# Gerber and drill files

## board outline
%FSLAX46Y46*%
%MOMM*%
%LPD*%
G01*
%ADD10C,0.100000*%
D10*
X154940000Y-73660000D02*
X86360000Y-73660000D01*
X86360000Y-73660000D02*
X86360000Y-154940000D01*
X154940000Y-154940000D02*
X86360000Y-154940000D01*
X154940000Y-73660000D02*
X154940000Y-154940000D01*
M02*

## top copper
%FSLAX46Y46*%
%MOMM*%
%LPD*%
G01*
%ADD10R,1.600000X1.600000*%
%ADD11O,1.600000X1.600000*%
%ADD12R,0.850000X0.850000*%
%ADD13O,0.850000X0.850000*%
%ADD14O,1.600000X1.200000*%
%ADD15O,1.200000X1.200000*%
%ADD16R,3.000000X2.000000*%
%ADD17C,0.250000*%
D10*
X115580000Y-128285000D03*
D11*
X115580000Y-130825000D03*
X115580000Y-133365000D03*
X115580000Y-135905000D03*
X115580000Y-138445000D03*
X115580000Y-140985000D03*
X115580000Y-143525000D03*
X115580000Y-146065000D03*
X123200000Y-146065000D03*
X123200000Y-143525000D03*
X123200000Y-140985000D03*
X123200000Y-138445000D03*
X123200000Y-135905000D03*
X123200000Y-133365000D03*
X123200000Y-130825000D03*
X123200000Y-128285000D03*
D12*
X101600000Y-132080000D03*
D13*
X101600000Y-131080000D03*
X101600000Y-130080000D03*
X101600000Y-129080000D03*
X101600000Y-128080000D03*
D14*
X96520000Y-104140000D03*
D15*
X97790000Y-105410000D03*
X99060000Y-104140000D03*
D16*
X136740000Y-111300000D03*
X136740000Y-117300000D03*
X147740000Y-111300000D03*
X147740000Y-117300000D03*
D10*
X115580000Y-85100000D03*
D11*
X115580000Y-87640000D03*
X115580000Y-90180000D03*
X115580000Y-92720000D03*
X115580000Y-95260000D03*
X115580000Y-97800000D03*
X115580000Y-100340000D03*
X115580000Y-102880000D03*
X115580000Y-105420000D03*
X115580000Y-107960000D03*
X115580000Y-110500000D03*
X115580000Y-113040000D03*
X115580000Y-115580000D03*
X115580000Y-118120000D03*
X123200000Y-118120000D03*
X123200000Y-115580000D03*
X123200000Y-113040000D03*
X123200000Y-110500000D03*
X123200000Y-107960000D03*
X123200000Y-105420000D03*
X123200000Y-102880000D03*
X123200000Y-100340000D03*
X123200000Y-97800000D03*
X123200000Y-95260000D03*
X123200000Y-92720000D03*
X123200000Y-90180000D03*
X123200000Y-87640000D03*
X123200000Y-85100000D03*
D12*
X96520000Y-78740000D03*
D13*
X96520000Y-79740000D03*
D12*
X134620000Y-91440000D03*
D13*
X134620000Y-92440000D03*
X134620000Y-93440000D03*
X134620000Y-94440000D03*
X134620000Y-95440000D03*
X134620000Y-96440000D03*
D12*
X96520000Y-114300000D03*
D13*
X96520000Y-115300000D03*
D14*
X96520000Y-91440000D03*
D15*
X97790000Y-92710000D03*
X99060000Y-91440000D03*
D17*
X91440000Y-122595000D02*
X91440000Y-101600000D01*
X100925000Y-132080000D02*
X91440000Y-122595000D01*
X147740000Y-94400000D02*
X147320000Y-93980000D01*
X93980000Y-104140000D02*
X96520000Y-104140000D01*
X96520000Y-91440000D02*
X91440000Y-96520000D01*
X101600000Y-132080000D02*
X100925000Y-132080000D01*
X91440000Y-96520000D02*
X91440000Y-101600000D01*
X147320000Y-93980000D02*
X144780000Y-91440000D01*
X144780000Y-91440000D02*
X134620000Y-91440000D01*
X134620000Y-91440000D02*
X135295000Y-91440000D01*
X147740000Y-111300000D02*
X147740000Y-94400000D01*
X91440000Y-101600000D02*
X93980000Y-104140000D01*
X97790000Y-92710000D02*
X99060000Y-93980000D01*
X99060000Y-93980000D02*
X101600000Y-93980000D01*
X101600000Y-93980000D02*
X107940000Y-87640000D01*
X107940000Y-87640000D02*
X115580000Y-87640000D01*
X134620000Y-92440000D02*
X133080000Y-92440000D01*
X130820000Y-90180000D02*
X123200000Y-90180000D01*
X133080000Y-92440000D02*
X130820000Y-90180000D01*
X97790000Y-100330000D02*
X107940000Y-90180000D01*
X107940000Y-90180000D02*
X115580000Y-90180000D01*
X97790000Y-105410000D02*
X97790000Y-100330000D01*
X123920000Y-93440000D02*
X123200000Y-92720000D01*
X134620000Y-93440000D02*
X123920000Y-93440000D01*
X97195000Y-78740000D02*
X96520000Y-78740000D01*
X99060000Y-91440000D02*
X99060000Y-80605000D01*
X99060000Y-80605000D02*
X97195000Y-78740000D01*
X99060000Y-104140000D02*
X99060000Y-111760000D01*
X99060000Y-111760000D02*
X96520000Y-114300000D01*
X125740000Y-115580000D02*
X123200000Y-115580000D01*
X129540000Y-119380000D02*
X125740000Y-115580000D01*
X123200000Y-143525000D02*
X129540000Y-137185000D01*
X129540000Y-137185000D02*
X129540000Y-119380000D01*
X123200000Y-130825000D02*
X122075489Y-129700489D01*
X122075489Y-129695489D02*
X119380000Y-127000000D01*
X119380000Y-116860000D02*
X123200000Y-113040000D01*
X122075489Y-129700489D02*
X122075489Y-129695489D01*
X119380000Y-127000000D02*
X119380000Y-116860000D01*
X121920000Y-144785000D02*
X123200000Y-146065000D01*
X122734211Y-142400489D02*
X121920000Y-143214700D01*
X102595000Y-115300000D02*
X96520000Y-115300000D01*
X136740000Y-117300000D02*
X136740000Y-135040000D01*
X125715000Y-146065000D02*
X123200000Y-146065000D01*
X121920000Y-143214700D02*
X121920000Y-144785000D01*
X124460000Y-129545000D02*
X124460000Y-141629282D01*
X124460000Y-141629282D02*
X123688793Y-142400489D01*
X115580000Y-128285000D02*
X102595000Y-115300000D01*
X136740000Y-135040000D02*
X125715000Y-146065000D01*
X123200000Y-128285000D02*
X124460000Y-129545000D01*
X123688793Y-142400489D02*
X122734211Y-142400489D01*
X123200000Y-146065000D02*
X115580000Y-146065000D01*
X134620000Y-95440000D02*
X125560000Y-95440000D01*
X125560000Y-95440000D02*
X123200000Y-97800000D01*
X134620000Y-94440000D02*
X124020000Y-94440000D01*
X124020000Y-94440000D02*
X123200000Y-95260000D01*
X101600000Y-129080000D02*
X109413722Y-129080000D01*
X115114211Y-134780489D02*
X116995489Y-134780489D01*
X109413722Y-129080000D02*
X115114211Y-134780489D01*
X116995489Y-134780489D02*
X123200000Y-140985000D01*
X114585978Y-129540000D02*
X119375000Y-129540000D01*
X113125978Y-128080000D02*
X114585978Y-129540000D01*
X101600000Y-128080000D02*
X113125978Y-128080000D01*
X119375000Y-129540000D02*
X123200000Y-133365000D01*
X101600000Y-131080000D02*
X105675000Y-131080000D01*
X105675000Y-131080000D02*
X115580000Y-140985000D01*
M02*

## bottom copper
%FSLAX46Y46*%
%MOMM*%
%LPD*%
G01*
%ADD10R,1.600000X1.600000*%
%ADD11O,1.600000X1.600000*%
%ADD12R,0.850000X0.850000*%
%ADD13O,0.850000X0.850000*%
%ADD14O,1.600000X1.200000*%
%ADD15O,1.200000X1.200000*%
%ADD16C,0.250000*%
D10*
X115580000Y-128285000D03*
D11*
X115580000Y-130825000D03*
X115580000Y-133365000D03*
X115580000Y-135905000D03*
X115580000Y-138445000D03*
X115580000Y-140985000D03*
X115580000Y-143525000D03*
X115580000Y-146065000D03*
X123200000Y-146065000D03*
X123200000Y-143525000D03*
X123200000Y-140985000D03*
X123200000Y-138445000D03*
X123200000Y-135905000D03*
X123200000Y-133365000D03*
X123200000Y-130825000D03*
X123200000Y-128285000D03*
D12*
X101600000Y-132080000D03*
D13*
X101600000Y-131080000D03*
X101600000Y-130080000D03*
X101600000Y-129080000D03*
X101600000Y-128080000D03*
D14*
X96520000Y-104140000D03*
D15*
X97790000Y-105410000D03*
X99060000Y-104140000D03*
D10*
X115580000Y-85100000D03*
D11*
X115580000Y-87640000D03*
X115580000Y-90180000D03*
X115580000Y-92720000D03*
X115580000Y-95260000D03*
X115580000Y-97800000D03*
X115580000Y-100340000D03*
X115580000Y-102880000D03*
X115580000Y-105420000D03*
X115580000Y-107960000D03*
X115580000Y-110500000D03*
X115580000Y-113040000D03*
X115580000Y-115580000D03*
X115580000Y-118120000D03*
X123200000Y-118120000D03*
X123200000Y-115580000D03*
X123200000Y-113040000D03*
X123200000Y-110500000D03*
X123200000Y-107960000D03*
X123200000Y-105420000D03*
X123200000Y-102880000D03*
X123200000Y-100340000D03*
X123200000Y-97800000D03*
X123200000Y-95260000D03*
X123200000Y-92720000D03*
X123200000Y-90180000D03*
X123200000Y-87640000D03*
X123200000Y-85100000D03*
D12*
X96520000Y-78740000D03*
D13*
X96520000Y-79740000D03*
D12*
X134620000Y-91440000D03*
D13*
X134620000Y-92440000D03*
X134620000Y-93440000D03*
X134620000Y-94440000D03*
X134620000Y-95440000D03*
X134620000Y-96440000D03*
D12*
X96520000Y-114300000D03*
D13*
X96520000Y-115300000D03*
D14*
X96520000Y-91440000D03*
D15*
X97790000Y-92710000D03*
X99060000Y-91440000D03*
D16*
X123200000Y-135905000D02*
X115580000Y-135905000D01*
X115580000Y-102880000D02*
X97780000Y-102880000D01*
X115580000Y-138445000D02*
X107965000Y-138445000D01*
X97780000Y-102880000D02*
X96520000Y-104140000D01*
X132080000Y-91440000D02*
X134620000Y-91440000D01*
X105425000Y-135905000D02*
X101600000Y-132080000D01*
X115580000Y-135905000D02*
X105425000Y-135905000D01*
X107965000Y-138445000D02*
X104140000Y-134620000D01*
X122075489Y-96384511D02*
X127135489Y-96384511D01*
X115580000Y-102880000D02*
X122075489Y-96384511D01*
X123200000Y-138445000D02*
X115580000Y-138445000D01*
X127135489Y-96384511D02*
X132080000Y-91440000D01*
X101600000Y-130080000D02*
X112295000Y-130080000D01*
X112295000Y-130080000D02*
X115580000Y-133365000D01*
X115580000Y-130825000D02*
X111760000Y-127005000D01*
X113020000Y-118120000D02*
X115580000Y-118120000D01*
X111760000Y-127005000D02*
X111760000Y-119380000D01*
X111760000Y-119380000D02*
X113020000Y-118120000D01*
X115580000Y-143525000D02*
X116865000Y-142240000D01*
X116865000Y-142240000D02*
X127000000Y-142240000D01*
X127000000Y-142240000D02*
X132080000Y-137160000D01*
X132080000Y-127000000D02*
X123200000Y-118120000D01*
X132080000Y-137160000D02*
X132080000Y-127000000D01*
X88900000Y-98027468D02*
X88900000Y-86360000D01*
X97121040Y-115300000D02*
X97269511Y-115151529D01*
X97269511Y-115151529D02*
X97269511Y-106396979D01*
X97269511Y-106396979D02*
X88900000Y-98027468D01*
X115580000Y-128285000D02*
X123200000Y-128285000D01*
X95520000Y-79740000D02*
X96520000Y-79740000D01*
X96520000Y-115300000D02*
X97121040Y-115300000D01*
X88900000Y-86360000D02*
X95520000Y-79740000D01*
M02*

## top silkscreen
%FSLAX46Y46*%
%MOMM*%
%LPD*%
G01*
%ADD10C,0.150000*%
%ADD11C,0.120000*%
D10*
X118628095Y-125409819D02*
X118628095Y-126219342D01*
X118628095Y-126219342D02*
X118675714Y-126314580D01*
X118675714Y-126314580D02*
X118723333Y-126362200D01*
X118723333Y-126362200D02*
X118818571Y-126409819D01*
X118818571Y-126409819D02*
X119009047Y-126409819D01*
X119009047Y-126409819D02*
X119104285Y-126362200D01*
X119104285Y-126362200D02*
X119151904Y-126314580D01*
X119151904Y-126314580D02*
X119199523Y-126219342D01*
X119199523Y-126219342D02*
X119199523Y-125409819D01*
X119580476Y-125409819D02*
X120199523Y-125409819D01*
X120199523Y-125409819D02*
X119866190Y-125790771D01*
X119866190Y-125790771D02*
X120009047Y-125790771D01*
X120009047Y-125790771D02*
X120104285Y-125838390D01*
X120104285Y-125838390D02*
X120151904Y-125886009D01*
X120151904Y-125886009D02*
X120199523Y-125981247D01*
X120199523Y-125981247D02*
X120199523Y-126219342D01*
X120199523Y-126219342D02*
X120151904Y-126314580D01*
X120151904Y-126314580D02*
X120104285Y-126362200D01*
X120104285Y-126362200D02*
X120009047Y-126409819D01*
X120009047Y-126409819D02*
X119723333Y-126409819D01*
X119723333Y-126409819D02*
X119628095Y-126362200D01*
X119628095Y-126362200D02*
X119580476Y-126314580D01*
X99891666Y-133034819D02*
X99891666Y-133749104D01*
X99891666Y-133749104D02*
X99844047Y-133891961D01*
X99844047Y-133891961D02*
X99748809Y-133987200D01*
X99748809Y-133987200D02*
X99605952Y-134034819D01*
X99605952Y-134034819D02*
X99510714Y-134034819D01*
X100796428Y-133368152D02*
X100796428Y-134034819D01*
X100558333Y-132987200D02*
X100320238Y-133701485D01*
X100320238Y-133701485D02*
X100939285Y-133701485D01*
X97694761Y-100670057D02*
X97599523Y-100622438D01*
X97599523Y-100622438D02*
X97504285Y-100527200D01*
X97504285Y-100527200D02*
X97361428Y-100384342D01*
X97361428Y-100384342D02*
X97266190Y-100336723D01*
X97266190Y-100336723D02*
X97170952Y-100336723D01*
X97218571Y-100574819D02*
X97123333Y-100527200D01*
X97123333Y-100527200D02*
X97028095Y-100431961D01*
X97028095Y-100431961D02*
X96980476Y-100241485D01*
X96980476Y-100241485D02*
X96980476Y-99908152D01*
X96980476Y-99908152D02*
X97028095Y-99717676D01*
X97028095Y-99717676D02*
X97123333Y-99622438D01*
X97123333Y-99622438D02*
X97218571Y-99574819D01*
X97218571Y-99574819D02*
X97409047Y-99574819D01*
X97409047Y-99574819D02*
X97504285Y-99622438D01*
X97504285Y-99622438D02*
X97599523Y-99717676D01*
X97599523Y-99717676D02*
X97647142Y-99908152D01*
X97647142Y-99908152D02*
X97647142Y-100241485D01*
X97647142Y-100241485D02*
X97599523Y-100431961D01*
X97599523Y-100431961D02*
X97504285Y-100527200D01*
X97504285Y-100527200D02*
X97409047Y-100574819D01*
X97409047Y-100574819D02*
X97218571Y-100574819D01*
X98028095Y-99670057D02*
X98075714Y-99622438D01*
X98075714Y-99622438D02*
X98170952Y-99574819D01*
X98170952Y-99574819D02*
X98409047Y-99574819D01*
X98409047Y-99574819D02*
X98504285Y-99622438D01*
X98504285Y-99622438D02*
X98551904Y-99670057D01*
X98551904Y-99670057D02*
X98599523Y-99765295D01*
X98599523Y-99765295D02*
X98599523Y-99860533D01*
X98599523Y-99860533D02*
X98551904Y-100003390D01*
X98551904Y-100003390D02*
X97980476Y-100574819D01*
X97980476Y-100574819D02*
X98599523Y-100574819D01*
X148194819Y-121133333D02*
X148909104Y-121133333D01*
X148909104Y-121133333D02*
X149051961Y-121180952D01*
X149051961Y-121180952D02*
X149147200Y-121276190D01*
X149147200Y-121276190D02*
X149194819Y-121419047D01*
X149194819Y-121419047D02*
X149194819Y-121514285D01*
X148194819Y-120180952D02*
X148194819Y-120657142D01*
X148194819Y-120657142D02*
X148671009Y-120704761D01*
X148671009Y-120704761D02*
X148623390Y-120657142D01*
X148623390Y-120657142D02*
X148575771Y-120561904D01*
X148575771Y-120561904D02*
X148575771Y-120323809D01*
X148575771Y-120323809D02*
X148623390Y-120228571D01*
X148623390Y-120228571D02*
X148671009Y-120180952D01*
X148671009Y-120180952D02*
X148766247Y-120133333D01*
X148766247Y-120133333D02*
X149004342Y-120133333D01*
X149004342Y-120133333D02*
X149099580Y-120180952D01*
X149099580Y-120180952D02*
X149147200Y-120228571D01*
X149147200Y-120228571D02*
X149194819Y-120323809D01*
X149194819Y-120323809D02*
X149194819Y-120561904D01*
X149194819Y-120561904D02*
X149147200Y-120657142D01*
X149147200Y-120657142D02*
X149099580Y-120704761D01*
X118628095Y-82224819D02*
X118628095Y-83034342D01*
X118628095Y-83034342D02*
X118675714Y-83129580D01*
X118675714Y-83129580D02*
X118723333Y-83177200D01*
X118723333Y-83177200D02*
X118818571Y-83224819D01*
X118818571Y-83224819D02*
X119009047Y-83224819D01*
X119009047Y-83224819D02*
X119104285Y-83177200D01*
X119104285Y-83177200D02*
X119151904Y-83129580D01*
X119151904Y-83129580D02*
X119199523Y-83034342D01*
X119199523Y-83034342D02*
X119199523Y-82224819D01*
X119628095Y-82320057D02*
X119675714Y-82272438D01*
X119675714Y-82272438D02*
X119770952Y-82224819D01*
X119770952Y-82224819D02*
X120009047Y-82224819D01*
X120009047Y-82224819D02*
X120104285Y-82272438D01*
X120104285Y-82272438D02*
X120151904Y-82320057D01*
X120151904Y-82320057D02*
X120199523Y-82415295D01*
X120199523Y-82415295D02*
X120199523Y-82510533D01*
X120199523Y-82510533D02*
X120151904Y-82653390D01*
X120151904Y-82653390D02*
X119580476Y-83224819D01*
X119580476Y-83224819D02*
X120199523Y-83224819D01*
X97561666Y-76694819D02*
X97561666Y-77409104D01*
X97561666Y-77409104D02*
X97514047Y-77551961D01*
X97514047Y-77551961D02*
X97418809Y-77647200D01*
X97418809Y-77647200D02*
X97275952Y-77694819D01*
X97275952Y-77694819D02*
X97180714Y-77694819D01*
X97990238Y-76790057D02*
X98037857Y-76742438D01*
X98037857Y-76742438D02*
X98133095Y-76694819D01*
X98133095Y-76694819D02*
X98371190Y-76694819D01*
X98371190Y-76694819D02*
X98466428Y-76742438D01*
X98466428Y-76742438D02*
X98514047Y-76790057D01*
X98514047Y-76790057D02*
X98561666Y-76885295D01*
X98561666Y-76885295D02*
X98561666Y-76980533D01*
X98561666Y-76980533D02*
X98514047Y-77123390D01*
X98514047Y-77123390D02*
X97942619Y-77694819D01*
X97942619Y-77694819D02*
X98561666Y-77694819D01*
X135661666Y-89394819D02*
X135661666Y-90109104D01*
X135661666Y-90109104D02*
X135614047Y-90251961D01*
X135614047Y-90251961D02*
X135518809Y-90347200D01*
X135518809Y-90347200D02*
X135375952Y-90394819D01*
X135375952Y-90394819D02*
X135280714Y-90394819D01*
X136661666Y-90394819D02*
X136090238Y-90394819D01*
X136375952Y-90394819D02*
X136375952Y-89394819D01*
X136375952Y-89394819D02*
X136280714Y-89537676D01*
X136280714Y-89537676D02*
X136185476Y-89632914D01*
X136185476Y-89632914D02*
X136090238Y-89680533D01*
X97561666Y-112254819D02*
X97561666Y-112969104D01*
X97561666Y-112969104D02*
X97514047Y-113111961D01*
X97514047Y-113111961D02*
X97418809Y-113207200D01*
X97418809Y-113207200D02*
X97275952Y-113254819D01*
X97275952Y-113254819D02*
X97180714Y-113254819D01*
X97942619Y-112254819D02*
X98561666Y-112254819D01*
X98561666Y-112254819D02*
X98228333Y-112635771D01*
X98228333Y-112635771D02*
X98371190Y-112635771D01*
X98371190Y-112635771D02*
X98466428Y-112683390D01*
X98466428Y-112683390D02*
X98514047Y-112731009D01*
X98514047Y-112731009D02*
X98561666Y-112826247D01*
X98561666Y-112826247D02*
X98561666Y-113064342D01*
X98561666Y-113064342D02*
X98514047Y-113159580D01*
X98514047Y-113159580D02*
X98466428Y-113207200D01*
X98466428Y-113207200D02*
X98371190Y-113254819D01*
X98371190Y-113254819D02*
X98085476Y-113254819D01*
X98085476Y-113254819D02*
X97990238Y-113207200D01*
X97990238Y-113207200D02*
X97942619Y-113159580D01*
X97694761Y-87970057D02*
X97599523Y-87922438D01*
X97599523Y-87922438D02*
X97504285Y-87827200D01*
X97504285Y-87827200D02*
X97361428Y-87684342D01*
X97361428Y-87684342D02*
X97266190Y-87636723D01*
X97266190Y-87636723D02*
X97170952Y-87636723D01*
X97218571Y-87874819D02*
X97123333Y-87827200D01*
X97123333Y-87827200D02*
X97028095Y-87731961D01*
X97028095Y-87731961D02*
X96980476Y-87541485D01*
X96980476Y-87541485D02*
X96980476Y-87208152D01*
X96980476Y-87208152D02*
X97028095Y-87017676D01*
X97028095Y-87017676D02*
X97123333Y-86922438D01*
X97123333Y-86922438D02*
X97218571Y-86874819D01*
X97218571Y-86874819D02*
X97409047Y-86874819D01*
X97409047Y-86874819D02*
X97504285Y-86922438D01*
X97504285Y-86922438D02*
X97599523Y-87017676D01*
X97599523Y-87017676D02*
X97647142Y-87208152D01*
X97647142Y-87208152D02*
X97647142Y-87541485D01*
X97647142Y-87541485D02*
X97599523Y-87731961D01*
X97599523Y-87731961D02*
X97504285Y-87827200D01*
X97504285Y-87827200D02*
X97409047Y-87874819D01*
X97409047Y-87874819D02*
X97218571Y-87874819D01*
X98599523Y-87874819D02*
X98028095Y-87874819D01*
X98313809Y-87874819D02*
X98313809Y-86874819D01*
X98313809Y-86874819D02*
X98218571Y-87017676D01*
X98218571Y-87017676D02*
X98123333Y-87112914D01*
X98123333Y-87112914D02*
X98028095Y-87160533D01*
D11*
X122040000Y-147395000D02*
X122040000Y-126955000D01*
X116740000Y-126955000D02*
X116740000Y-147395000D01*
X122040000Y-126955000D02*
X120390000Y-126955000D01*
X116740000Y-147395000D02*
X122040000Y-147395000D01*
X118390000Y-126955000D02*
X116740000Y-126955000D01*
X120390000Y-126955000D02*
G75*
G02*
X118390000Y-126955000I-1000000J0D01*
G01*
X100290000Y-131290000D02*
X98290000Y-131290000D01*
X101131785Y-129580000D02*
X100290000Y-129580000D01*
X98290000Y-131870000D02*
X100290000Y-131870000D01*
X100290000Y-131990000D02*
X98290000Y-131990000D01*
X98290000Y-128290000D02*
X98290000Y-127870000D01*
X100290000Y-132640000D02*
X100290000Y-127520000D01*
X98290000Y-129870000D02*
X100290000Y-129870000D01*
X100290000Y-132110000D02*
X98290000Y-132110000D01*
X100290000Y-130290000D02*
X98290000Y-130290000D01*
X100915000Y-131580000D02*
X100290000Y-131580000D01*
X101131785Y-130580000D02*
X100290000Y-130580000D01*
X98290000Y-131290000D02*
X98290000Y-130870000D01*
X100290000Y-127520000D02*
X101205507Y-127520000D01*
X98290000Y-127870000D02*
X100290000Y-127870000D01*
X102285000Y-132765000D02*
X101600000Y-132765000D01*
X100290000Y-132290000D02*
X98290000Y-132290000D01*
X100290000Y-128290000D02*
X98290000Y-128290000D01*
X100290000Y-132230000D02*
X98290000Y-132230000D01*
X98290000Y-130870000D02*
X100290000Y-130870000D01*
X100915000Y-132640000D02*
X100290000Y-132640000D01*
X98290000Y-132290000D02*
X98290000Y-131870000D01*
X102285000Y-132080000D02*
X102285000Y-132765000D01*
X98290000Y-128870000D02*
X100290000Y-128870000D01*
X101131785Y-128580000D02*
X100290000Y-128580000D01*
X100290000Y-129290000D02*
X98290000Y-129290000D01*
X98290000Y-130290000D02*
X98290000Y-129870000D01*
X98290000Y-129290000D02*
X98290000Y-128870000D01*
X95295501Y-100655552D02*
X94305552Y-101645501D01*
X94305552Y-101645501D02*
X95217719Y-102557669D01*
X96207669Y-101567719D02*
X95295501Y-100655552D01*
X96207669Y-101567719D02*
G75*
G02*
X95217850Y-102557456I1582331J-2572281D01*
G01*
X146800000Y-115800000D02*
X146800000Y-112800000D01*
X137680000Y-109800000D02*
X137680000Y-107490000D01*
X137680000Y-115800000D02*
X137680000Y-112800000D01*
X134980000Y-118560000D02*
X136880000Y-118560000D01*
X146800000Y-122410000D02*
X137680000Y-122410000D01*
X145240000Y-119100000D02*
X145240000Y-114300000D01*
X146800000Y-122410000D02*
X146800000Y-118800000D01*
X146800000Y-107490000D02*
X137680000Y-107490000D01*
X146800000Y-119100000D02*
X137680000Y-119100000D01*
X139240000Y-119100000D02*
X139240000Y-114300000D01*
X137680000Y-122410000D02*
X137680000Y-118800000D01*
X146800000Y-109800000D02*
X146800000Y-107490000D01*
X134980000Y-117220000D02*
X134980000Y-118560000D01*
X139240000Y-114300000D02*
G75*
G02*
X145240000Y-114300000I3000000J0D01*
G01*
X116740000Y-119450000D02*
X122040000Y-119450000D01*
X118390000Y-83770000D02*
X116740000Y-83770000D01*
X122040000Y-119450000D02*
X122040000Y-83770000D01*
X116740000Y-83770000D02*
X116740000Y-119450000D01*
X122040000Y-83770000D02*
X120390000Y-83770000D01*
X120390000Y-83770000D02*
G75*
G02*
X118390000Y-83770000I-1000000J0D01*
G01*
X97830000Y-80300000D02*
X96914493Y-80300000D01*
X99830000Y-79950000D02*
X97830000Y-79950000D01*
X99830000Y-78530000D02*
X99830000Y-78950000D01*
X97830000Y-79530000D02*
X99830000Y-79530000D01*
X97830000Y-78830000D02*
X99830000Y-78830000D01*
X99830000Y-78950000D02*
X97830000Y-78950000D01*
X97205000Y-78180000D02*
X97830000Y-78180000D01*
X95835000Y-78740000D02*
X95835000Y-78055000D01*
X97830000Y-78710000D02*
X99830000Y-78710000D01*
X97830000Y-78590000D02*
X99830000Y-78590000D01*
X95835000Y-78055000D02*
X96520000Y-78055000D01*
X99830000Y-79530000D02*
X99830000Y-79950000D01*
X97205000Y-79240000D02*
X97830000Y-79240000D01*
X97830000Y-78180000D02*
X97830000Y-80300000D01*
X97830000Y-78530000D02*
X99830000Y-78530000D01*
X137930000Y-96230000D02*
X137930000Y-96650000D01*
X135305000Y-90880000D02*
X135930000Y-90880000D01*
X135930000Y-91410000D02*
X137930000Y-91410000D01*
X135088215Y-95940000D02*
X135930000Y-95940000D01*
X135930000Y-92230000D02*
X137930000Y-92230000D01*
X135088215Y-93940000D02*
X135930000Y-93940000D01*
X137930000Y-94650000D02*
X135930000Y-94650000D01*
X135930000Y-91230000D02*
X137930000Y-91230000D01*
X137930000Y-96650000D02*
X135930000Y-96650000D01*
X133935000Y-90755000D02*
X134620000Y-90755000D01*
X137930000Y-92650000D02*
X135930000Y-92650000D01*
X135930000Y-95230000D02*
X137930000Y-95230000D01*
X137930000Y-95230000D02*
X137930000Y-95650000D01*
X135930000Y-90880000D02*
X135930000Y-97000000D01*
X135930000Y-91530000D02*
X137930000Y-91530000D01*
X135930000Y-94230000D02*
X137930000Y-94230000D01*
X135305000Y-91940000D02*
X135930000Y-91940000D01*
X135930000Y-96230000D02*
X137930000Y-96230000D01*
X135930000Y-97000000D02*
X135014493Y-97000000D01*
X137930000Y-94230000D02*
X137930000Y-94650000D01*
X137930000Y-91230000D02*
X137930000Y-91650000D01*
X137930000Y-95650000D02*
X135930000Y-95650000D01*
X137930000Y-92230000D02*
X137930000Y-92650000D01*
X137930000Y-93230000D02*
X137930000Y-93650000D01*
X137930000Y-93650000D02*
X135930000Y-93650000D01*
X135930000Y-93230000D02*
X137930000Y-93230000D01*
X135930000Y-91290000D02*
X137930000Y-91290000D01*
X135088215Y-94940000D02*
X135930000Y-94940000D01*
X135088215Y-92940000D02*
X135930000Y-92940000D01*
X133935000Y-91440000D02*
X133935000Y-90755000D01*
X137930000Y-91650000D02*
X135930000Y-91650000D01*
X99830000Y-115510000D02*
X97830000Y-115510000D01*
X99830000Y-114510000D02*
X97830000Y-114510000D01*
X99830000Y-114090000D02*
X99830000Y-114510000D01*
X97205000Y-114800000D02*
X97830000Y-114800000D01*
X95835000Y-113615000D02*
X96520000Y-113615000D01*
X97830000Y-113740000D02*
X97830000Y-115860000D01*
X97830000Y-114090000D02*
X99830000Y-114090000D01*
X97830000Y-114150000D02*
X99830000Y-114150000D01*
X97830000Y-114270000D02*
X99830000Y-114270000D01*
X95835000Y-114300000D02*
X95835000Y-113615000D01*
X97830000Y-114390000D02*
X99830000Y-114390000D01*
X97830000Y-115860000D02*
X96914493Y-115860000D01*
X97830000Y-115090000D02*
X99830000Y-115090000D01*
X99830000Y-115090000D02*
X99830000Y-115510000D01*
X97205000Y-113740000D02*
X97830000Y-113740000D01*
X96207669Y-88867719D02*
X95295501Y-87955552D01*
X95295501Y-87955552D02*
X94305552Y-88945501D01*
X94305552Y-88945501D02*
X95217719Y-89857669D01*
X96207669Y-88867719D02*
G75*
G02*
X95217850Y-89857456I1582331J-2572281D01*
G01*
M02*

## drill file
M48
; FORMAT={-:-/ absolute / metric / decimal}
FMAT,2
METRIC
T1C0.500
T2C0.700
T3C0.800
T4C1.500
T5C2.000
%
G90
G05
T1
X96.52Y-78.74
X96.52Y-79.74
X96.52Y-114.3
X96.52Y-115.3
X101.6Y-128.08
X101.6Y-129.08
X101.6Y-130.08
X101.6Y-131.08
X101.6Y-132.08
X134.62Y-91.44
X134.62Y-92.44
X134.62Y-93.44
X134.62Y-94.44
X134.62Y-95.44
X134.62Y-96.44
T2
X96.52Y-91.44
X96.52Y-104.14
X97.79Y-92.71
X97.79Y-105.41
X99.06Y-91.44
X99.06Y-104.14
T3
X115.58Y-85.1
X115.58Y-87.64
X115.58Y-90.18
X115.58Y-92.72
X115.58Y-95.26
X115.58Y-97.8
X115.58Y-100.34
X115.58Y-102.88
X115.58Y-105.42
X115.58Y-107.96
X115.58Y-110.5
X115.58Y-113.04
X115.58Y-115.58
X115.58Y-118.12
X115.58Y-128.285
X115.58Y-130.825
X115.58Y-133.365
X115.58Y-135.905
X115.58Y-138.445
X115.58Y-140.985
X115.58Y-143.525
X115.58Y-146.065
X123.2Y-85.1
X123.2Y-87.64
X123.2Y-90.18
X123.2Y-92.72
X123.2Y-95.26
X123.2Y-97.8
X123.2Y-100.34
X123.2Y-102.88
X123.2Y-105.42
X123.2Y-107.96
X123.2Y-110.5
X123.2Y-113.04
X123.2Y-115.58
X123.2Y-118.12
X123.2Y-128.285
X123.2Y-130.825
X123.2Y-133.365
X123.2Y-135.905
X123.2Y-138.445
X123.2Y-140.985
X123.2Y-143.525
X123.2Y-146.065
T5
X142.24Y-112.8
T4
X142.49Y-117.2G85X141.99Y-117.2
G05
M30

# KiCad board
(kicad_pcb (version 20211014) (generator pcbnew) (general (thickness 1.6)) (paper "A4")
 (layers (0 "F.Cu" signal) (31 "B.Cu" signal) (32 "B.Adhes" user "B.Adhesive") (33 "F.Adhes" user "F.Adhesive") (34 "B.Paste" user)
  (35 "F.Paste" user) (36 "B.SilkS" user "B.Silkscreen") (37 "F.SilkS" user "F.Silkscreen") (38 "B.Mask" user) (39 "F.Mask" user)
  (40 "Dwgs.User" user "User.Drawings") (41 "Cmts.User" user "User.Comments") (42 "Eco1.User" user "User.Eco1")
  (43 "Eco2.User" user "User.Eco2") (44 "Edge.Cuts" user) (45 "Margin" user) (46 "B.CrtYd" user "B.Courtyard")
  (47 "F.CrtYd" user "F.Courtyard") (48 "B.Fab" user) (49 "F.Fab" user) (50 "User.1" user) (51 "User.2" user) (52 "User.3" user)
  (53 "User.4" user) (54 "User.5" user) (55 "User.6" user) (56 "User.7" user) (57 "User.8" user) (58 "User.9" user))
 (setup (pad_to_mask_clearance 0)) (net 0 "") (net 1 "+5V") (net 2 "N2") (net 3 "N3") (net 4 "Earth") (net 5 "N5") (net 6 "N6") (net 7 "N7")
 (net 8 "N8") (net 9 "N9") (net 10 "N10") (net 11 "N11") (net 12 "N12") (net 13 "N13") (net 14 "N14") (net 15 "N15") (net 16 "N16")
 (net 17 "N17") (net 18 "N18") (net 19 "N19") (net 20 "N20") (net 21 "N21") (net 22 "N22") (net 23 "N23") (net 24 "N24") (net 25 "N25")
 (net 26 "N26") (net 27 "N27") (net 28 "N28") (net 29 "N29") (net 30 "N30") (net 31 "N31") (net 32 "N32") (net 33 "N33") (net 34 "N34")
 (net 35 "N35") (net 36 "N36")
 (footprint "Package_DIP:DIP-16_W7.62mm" (layer "F.Cu") (at 115.58 128.285)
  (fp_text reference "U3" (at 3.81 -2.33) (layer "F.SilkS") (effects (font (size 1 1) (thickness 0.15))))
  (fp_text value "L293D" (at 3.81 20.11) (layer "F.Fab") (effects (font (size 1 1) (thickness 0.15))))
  (fp_line (start 6.46 19.11) (end 6.46 -1.33) (layer "F.SilkS") (width 0.12))
  (fp_line (start 1.16 -1.33) (end 1.16 19.11) (layer "F.SilkS") (width 0.12))
  (fp_line (start 6.46 -1.33) (end 4.81 -1.33) (layer "F.SilkS") (width 0.12))
  (fp_line (start 1.16 19.11) (end 6.46 19.11) (layer "F.SilkS") (width 0.12))
  (fp_line (start 2.81 -1.33) (end 1.16 -1.33) (layer "F.SilkS") (width 0.12))
  (fp_arc (start 4.81 -1.33) (mid 3.81 -0.33) (end 2.81 -1.33) (layer "F.SilkS") (width 0.12))
  (pad "1" thru_hole rect (at 0 0) (size 1.6 1.6) (drill 0.8) (layers *.Cu *.Mask) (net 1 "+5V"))
  (pad "2" thru_hole oval (at 0 2.54) (size 1.6 1.6) (drill 0.8) (layers *.Cu *.Mask) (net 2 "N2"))
  (pad "3" thru_hole oval (at 0 5.08) (size 1.6 1.6) (drill 0.8) (layers *.Cu *.Mask) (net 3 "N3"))
  (pad "4" thru_hole oval (at 0 7.62) (size 1.6 1.6) (drill 0.8) (layers *.Cu *.Mask) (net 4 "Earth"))
  (pad "5" thru_hole oval (at 0 10.16) (size 1.6 1.6) (drill 0.8) (layers *.Cu *.Mask) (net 4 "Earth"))
  (pad "6" thru_hole oval (at 0 12.7) (size 1.6 1.6) (drill 0.8) (layers *.Cu *.Mask) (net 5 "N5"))
  (pad "7" thru_hole oval (at 0 15.24) (size 1.6 1.6) (drill 0.8) (layers *.Cu *.Mask) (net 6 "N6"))
  (pad "8" thru_hole oval (at 0 17.78) (size 1.6 1.6) (drill 0.8) (layers *.Cu *.Mask) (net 1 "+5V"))
  (pad "9" thru_hole oval (at 7.62 17.78) (size 1.6 1.6) (drill 0.8) (layers *.Cu *.Mask) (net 1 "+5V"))
  (pad "10" thru_hole oval (at 7.62 15.24) (size 1.6 1.6) (drill 0.8) (layers *.Cu *.Mask) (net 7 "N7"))
  (pad "11" thru_hole oval (at 7.62 12.7) (size 1.6 1.6) (drill 0.8) (layers *.Cu *.Mask) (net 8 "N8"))
  (pad "12" thru_hole oval (at 7.62 10.16) (size 1.6 1.6) (drill 0.8) (layers *.Cu *.Mask) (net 4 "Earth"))
  (pad "13" thru_hole oval (at 7.62 7.62) (size 1.6 1.6) (drill 0.8) (layers *.Cu *.Mask) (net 4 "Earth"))
  (pad "14" thru_hole oval (at 7.62 5.08) (size 1.6 1.6) (drill 0.8) (layers *.Cu *.Mask) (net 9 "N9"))
  (pad "15" thru_hole oval (at 7.62 2.54) (size 1.6 1.6) (drill 0.8) (layers *.Cu *.Mask) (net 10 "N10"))
  (pad "16" thru_hole oval (at 7.62 0) (size 1.6 1.6) (drill 0.8) (layers *.Cu *.Mask) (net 1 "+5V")))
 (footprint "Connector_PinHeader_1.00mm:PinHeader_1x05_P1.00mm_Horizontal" (layer "F.Cu") (at 101.6 132.08 180)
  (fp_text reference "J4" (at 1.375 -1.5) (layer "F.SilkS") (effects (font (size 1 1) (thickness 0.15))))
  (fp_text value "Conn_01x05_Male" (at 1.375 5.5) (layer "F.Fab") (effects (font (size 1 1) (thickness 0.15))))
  (fp_line (start 1.31 0.79) (end 3.31 0.79) (layer "F.SilkS") (width 0.12))
  (fp_line (start 0.468215 2.5) (end 1.31 2.5) (layer "F.SilkS") (width 0.12))
  (fp_line (start 3.31 0.21) (end 1.31 0.21) (layer "F.SilkS") (width 0.12))
  (fp_line (start 1.31 0.09) (end 3.31 0.09) (layer "F.SilkS") (width 0.12))
  (fp_line (start 3.31 3.79) (end 3.31 4.21) (layer "F.SilkS") (width 0.12))
  (fp_line (start 1.31 -0.56) (end 1.31 4.56) (layer "F.SilkS") (width 0.12))
  (fp_line (start 3.31 2.21) (end 1.31 2.21) (layer "F.SilkS") (width 0.12))
  (fp_line (start 1.31 -0.03) (end 3.31 -0.03) (layer "F.SilkS") (width 0.12))
  (fp_line (start 1.31 1.79) (end 3.31 1.79) (layer "F.SilkS") (width 0.12))
  (fp_line (start 0.685 0.5) (end 1.31 0.5) (layer "F.SilkS") (width 0.12))
  (fp_line (start 0.468215 1.5) (end 1.31 1.5) (layer "F.SilkS") (width 0.12))
  (fp_line (start 3.31 0.79) (end 3.31 1.21) (layer "F.SilkS") (width 0.12))
  (fp_line (start 1.31 4.56) (end 0.394493 4.56) (layer "F.SilkS") (width 0.12))
  (fp_line (start 3.31 4.21) (end 1.31 4.21) (layer "F.SilkS") (width 0.12))
  (fp_line (start -0.685 -0.685) (end 0 -0.685) (layer "F.SilkS") (width 0.12))
  (fp_line (start 1.31 -0.21) (end 3.31 -0.21) (layer "F.SilkS") (width 0.12))
  (fp_line (start 1.31 3.79) (end 3.31 3.79) (layer "F.SilkS") (width 0.12))
  (fp_line (start 1.31 -0.15) (end 3.31 -0.15) (layer "F.SilkS") (width 0.12))
  (fp_line (start 3.31 1.21) (end 1.31 1.21) (layer "F.SilkS") (width 0.12))
  (fp_line (start 0.685 -0.56) (end 1.31 -0.56) (layer "F.SilkS") (width 0.12))
  (fp_line (start 3.31 -0.21) (end 3.31 0.21) (layer "F.SilkS") (width 0.12))
  (fp_line (start -0.685 0) (end -0.685 -0.685) (layer "F.SilkS") (width 0.12))
  (fp_line (start 3.31 3.21) (end 1.31 3.21) (layer "F.SilkS") (width 0.12))
  (fp_line (start 0.468215 3.5) (end 1.31 3.5) (layer "F.SilkS") (width 0.12))
  (fp_line (start 1.31 2.79) (end 3.31 2.79) (layer "F.SilkS") (width 0.12))
  (fp_line (start 3.31 1.79) (end 3.31 2.21) (layer "F.SilkS") (width 0.12))
  (fp_line (start 3.31 2.79) (end 3.31 3.21) (layer "F.SilkS") (width 0.12))
  (pad "1" thru_hole rect (at 0 0 180) (size 0.85 0.85) (drill 0.5) (layers *.Cu *.Mask) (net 4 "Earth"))
  (pad "2" thru_hole oval (at 0 1 180) (size 0.85 0.85) (drill 0.5) (layers *.Cu *.Mask) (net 5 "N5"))
  (pad "3" thru_hole oval (at 0 2 180) (size 0.85 0.85) (drill 0.5) (layers *.Cu *.Mask) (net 3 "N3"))
  (pad "4" thru_hole oval (at 0 3 180) (size 0.85 0.85) (drill 0.5) (layers *.Cu *.Mask) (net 8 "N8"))
  (pad "5" thru_hole oval (at 0 4 180) (size 0.85 0.85) (drill 0.5) (layers *.Cu *.Mask) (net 9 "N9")))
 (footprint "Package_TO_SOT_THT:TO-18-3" (layer "F.Cu") (at 96.52 104.14)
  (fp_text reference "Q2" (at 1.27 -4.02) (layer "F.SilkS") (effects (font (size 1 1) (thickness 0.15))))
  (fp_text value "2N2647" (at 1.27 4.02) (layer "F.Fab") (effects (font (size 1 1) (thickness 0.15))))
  (fp_line (start -1.224499 -3.484448) (end -2.214448 -2.494499) (layer "F.SilkS") (width 0.12))
  (fp_line (start -2.214448 -2.494499) (end -1.302281 -1.582331) (layer "F.SilkS") (width 0.12))
  (fp_line (start -0.312331 -2.572281) (end -1.224499 -3.484448) (layer "F.SilkS") (width 0.12))
  (fp_arc (start -0.312331 -2.572281) (mid 3.405374 2.135551) (end -1.30215 -1.582544) (layer "F.SilkS") (width 0.12))
  (pad "1" thru_hole oval (at 0 0) (size 1.6 1.2) (drill 0.7) (layers *.Cu *.Mask) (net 4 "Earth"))
  (pad "2" thru_hole oval (at 1.27 1.27) (size 1.2 1.2) (drill 0.7) (layers *.Cu *.Mask) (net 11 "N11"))
  (pad "3" thru_hole oval (at 2.54 0) (size 1.2 1.2) (drill 0.7) (layers *.Cu *.Mask) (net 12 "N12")))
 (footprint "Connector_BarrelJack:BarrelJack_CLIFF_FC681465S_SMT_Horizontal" (layer "F.Cu") (at 142.24 114.3 90)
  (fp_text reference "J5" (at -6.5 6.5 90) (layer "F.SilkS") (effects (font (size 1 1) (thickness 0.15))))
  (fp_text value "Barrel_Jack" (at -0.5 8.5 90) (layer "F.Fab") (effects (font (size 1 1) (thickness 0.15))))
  (fp_line (start -1.5 4.56) (end 1.5 4.56) (layer "F.SilkS") (width 0.12))
  (fp_line (start 4.5 -4.56) (end 6.81 -4.56) (layer "F.SilkS") (width 0.12))
  (fp_line (start -1.5 -4.56) (end 1.5 -4.56) (layer "F.SilkS") (width 0.12))
  (fp_line (start -4.26 -7.26) (end -4.26 -5.36) (layer "F.SilkS") (width 0.12))
  (fp_line (start -8.11 4.56) (end -8.11 -4.56) (layer "F.SilkS") (width 0.12))
  (fp_line (start -4.8 3) (end 0 3) (layer "F.SilkS") (width 0.12))
  (fp_line (start -8.11 4.56) (end -4.5 4.56) (layer "F.SilkS") (width 0.12))
  (fp_line (start 6.81 4.56) (end 6.81 -4.56) (layer "F.SilkS") (width 0.12))
  (fp_line (start -4.8 4.56) (end -4.8 -4.56) (layer "F.SilkS") (width 0.12))
  (fp_line (start -4.8 -3) (end 0 -3) (layer "F.SilkS") (width 0.12))
  (fp_line (start -8.11 -4.56) (end -4.5 -4.56) (layer "F.SilkS") (width 0.12))
  (fp_line (start 4.5 4.56) (end 6.81 4.56) (layer "F.SilkS") (width 0.12))
  (fp_line (start -2.92 -7.26) (end -4.26 -7.26) (layer "F.SilkS") (width 0.12))
  (fp_arc (start 0 -3) (mid 3 0) (end 0 3) (layer "F.SilkS") (width 0.12))
  (pad "" np_thru_hole circle (at 1.5 0 180) (size 2 2) (drill 2) (layers *.Cu *.Mask))
  (pad "" np_thru_hole oval (at -2.9 0 180) (size 2 1.5) (drill oval 2 1.5) (layers *.Cu *.Mask))
  (pad "1" smd rect (at 3 -5.5 180) (size 3 2) (layers "F.Cu" "F.Paste" "F.Mask") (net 1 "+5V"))
  (pad "1" smd rect (at -3 -5.5 180) (size 3 2) (layers "F.Cu" "F.Paste" "F.Mask") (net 1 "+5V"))
  (pad "2" smd rect (at 3 5.5 180) (size 3 2) (layers "F.Cu" "F.Paste" "F.Mask") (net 4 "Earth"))
  (pad "3" smd rect (at -3 5.5 180) (size 3 2) (layers "F.Cu" "F.Paste" "F.Mask")))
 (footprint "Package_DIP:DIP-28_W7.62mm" (layer "F.Cu") (at 115.58 85.1)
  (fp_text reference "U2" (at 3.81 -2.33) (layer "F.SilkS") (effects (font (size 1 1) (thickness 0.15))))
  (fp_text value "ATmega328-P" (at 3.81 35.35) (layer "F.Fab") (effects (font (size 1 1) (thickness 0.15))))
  (fp_line (start 1.16 34.35) (end 6.46 34.35) (layer "F.SilkS") (width 0.12))
  (fp_line (start 2.81 -1.33) (end 1.16 -1.33) (layer "F.SilkS") (width 0.12))
  (fp_line (start 6.46 34.35) (end 6.46 -1.33) (layer "F.SilkS") (width 0.12))
  (fp_line (start 1.16 -1.33) (end 1.16 34.35) (layer "F.SilkS") (width 0.12))
  (fp_line (start 6.46 -1.33) (end 4.81 -1.33) (layer "F.SilkS") (width 0.12))
  (fp_arc (start 4.81 -1.33) (mid 3.81 -0.33) (end 2.81 -1.33) (layer "F.SilkS") (width 0.12))
  (pad "1" thru_hole rect (at 0 0) (size 1.6 1.6) (drill 0.8) (layers *.Cu *.Mask) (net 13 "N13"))
  (pad "2" thru_hole oval (at 0 2.54) (size 1.6 1.6) (drill 0.8) (layers *.Cu *.Mask) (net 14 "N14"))
  (pad "3" thru_hole oval (at 0 5.08) (size 1.6 1.6) (drill 0.8) (layers *.Cu *.Mask) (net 11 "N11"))
  (pad "4" thru_hole oval (at 0 7.62) (size 1.6 1.6) (drill 0.8) (layers *.Cu *.Mask) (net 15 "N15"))
  (pad "5" thru_hole oval (at 0 10.16) (size 1.6 1.6) (drill 0.8) (layers *.Cu *.Mask) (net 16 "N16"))
  (pad "6" thru_hole oval (at 0 12.7) (size 1.6 1.6) (drill 0.8) (layers *.Cu *.Mask) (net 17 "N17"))
  (pad "7" thru_hole oval (at 0 15.24) (size 1.6 1.6) (drill 0.8) (layers *.Cu *.Mask) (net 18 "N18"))
  (pad "8" thru_hole oval (at 0 17.78) (size 1.6 1.6) (drill 0.8) (layers *.Cu *.Mask) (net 4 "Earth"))
  (pad "9" thru_hole oval (at 0 20.32) (size 1.6 1.6) (drill 0.8) (layers *.Cu *.Mask) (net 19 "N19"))
  (pad "10" thru_hole oval (at 0 22.86) (size 1.6 1.6) (drill 0.8) (layers *.Cu *.Mask) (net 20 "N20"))
  (pad "11" thru_hole oval (at 0 25.4) (size 1.6 1.6) (drill 0.8) (layers *.Cu *.Mask) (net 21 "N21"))
  (pad "12" thru_hole oval (at 0 27.94) (size 1.6 1.6) (drill 0.8) (layers *.Cu *.Mask) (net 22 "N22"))
  (pad "13" thru_hole oval (at 0 30.48) (size 1.6 1.6) (drill 0.8) (layers *.Cu *.Mask) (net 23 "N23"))
  (pad "14" thru_hole oval (at 0 33.02) (size 1.6 1.6) (drill 0.8) (layers *.Cu *.Mask) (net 2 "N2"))
  (pad "15" thru_hole oval (at 7.62 33.02) (size 1.6 1.6) (drill 0.8) (layers *.Cu *.Mask) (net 6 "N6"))
  (pad "16" thru_hole oval (at 7.62 30.48) (size 1.6 1.6) (drill 0.8) (layers *.Cu *.Mask) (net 7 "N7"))
  (pad "17" thru_hole oval (at 7.62 27.94) (size 1.6 1.6) (drill 0.8) (layers *.Cu *.Mask) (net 10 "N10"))
  (pad "18" thru_hole oval (at 7.62 25.4) (size 1.6 1.6) (drill 0.8) (layers *.Cu *.Mask) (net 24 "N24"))
  (pad "19" thru_hole oval (at 7.62 22.86) (size 1.6 1.6) (drill 0.8) (layers *.Cu *.Mask) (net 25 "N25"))
  (pad "20" thru_hole oval (at 7.62 20.32) (size 1.6 1.6) (drill 0.8) (layers *.Cu *.Mask) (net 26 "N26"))
  (pad "21" thru_hole oval (at 7.62 17.78) (size 1.6 1.6) (drill 0.8) (layers *.Cu *.Mask) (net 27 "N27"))
  (pad "22" thru_hole oval (at 7.62 15.24) (size 1.6 1.6) (drill 0.8) (layers *.Cu *.Mask) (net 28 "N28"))
  (pad "23" thru_hole oval (at 7.62 12.7) (size 1.6 1.6) (drill 0.8) (layers *.Cu *.Mask) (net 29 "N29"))
  (pad "24" thru_hole oval (at 7.62 10.16) (size 1.6 1.6) (drill 0.8) (layers *.Cu *.Mask) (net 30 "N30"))
  (pad "25" thru_hole oval (at 7.62 7.62) (size 1.6 1.6) (drill 0.8) (layers *.Cu *.Mask) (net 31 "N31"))
  (pad "26" thru_hole oval (at 7.62 5.08) (size 1.6 1.6) (drill 0.8) (layers *.Cu *.Mask) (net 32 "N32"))
  (pad "27" thru_hole oval (at 7.62 2.54) (size 1.6 1.6) (drill 0.8) (layers *.Cu *.Mask) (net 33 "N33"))
  (pad "28" thru_hole oval (at 7.62 0) (size 1.6 1.6) (drill 0.8) (layers *.Cu *.Mask) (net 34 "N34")))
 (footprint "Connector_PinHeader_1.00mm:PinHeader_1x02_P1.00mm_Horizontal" (layer "F.Cu") (at 96.52 78.74)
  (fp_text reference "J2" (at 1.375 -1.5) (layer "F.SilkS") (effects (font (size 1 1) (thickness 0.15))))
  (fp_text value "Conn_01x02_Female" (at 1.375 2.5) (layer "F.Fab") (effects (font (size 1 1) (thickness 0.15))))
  (fp_line (start 1.31 1.56) (end 0.394493 1.56) (layer "F.SilkS") (width 0.12))
  (fp_line (start 3.31 1.21) (end 1.31 1.21) (layer "F.SilkS") (width 0.12))
  (fp_line (start 3.31 -0.21) (end 3.31 0.21) (layer "F.SilkS") (width 0.12))
  (fp_line (start 1.31 0.79) (end 3.31 0.79) (layer "F.SilkS") (width 0.12))
  (fp_line (start 1.31 0.09) (end 3.31 0.09) (layer "F.SilkS") (width 0.12))
  (fp_line (start 3.31 0.21) (end 1.31 0.21) (layer "F.SilkS") (width 0.12))
  (fp_line (start 0.685 -0.56) (end 1.31 -0.56) (layer "F.SilkS") (width 0.12))
  (fp_line (start -0.685 0) (end -0.685 -0.685) (layer "F.SilkS") (width 0.12))
  (fp_line (start 1.31 -0.03) (end 3.31 -0.03) (layer "F.SilkS") (width 0.12))
  (fp_line (start 1.31 -0.15) (end 3.31 -0.15) (layer "F.SilkS") (width 0.12))
  (fp_line (start -0.685 -0.685) (end 0 -0.685) (layer "F.SilkS") (width 0.12))
  (fp_line (start 3.31 0.79) (end 3.31 1.21) (layer "F.SilkS") (width 0.12))
  (fp_line (start 0.685 0.5) (end 1.31 0.5) (layer "F.SilkS") (width 0.12))
  (fp_line (start 1.31 -0.56) (end 1.31 1.56) (layer "F.SilkS") (width 0.12))
  (fp_line (start 1.31 -0.21) (end 3.31 -0.21) (layer "F.SilkS") (width 0.12))
  (pad "1" thru_hole rect (at 0 0) (size 0.85 0.85) (drill 0.5) (layers *.Cu *.Mask) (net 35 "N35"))
  (pad "2" thru_hole oval (at 0 1) (size 0.85 0.85) (drill 0.5) (layers *.Cu *.Mask) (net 1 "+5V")))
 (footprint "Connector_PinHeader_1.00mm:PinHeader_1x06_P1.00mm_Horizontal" (layer "F.Cu") (at 134.62 91.44)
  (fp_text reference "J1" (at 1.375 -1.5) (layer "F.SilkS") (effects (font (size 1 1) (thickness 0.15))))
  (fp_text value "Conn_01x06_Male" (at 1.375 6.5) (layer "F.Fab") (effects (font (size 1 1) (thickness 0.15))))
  (fp_line (start 3.31 4.79) (end 3.31 5.21) (layer "F.SilkS") (width 0.12))
  (fp_line (start 0.685 -0.56) (end 1.31 -0.56) (layer "F.SilkS") (width 0.12))
  (fp_line (start 1.31 -0.03) (end 3.31 -0.03) (layer "F.SilkS") (width 0.12))
  (fp_line (start 0.468215 4.5) (end 1.31 4.5) (layer "F.SilkS") (width 0.12))
  (fp_line (start 1.31 0.79) (end 3.31 0.79) (layer "F.SilkS") (width 0.12))
  (fp_line (start 0.468215 2.5) (end 1.31 2.5) (layer "F.SilkS") (width 0.12))
  (fp_line (start 3.31 3.21) (end 1.31 3.21) (layer "F.SilkS") (width 0.12))
  (fp_line (start 1.31 -0.21) (end 3.31 -0.21) (layer "F.SilkS") (width 0.12))
  (fp_line (start 3.31 5.21) (end 1.31 5.21) (layer "F.SilkS") (width 0.12))
  (fp_line (start -0.685 -0.685) (end 0 -0.685) (layer "F.SilkS") (width 0.12))
  (fp_line (start 3.31 1.21) (end 1.31 1.21) (layer "F.SilkS") (width 0.12))
  (fp_line (start 1.31 3.79) (end 3.31 3.79) (layer "F.SilkS") (width 0.12))
  (fp_line (start 3.31 3.79) (end 3.31 4.21) (layer "F.SilkS") (width 0.12))
  (fp_line (start 1.31 -0.56) (end 1.31 5.56) (layer "F.SilkS") (width 0.12))
  (fp_line (start 1.31 0.09) (end 3.31 0.09) (layer "F.SilkS") (width 0.12))
  (fp_line (start 1.31 2.79) (end 3.31 2.79) (layer "F.SilkS") (width 0.12))
  (fp_line (start 0.685 0.5) (end 1.31 0.5) (layer "F.SilkS") (width 0.12))
  (fp_line (start 1.31 4.79) (end 3.31 4.79) (layer "F.SilkS") (width 0.12))
  (fp_line (start 1.31 5.56) (end 0.394493 5.56) (layer "F.SilkS") (width 0.12))
  (fp_line (start 3.31 2.79) (end 3.31 3.21) (layer "F.SilkS") (width 0.12))
  (fp_line (start 3.31 -0.21) (end 3.31 0.21) (layer "F.SilkS") (width 0.12))
  (fp_line (start 3.31 4.21) (end 1.31 4.21) (layer "F.SilkS") (width 0.12))
  (fp_line (start 3.31 0.79) (end 3.31 1.21) (layer "F.SilkS") (width 0.12))
  (fp_line (start 3.31 1.79) (end 3.31 2.21) (layer "F.SilkS") (width 0.12))
  (fp_line (start 3.31 2.21) (end 1.31 2.21) (layer "F.SilkS") (width 0.12))
  (fp_line (start 1.31 1.79) (end 3.31 1.79) (layer "F.SilkS") (width 0.12))
  (fp_line (start 1.31 -0.15) (end 3.31 -0.15) (layer "F.SilkS") (width 0.12))
  (fp_line (start 0.468215 3.5) (end 1.31 3.5) (layer "F.SilkS") (width 0.12))
  (fp_line (start 0.468215 1.5) (end 1.31 1.5) (layer "F.SilkS") (width 0.12))
  (fp_line (start -0.685 0) (end -0.685 -0.685) (layer "F.SilkS") (width 0.12))
  (fp_line (start 3.31 0.21) (end 1.31 0.21) (layer "F.SilkS") (width 0.12))
  (pad "1" thru_hole rect (at 0 0) (size 0.85 0.85) (drill 0.5) (layers *.Cu *.Mask) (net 4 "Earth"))
  (pad "2" thru_hole oval (at 0 1) (size 0.85 0.85) (drill 0.5) (layers *.Cu *.Mask) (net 32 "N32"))
  (pad "3" thru_hole oval (at 0 2) (size 0.85 0.85) (drill 0.5) (layers *.Cu *.Mask) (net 31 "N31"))
  (pad "4" thru_hole oval (at 0 3) (size 0.85 0.85) (drill 0.5) (layers *.Cu *.Mask) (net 30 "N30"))
  (pad "5" thru_hole oval (at 0 4) (size 0.85 0.85) (drill 0.5) (layers *.Cu *.Mask) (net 29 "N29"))
  (pad "6" thru_hole oval (at 0 5) (size 0.85 0.85) (drill 0.5) (layers *.Cu *.Mask) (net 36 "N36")))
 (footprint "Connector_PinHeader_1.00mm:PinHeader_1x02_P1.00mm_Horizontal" (layer "F.Cu") (at 96.52 114.3)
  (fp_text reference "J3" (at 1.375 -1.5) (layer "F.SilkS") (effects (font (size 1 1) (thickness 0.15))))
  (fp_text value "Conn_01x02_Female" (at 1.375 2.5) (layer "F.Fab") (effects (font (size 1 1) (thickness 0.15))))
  (fp_line (start 3.31 1.21) (end 1.31 1.21) (layer "F.SilkS") (width 0.12))
  (fp_line (start 3.31 0.21) (end 1.31 0.21) (layer "F.SilkS") (width 0.12))
  (fp_line (start 3.31 -0.21) (end 3.31 0.21) (layer "F.SilkS") (width 0.12))
  (fp_line (start 0.685 0.5) (end 1.31 0.5) (layer "F.SilkS") (width 0.12))
  (fp_line (start -0.685 -0.685) (end 0 -0.685) (layer "F.SilkS") (width 0.12))
  (fp_line (start 1.31 -0.56) (end 1.31 1.56) (layer "F.SilkS") (width 0.12))
  (fp_line (start 1.31 -0.21) (end 3.31 -0.21) (layer "F.SilkS") (width 0.12))
  (fp_line (start 1.31 -0.15) (end 3.31 -0.15) (layer "F.SilkS") (width 0.12))
  (fp_line (start 1.31 -0.03) (end 3.31 -0.03) (layer "F.SilkS") (width 0.12))
  (fp_line (start -0.685 0) (end -0.685 -0.685) (layer "F.SilkS") (width 0.12))
  (fp_line (start 1.31 0.09) (end 3.31 0.09) (layer "F.SilkS") (width 0.12))
  (fp_line (start 1.31 1.56) (end 0.394493 1.56) (layer "F.SilkS") (width 0.12))
  (fp_line (start 1.31 0.79) (end 3.31 0.79) (layer "F.SilkS") (width 0.12))
  (fp_line (start 3.31 0.79) (end 3.31 1.21) (layer "F.SilkS") (width 0.12))
  (fp_line (start 0.685 -0.56) (end 1.31 -0.56) (layer "F.SilkS") (width 0.12))
  (pad "1" thru_hole rect (at 0 0) (size 0.85 0.85) (drill 0.5) (layers *.Cu *.Mask) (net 12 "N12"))
  (pad "2" thru_hole oval (at 0 1) (size 0.85 0.85) (drill 0.5) (layers *.Cu *.Mask) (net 1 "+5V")))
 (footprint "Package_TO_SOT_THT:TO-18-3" (layer "F.Cu") (at 96.52 91.44)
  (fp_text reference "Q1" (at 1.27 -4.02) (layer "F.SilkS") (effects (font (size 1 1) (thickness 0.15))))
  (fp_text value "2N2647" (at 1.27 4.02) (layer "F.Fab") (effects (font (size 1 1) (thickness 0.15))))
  (fp_line (start -0.312331 -2.572281) (end -1.224499 -3.484448) (layer "F.SilkS") (width 0.12))
  (fp_line (start -1.224499 -3.484448) (end -2.214448 -2.494499) (layer "F.SilkS") (width 0.12))
  (fp_line (start -2.214448 -2.494499) (end -1.302281 -1.582331) (layer "F.SilkS") (width 0.12))
  (fp_arc (start -0.312331 -2.572281) (mid 3.405374 2.135551) (end -1.30215 -1.582544) (layer "F.SilkS") (width 0.12))
  (pad "1" thru_hole oval (at 0 0) (size 1.6 1.2) (drill 0.7) (layers *.Cu *.Mask) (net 4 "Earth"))
  (pad "2" thru_hole oval (at 1.27 1.27) (size 1.2 1.2) (drill 0.7) (layers *.Cu *.Mask) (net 14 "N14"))
  (pad "3" thru_hole oval (at 2.54 0) (size 1.2 1.2) (drill 0.7) (layers *.Cu *.Mask) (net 35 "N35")))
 (gr_line (start 154.94 73.66) (end 86.36 73.66) (layer "Edge.Cuts") (width 0.1))
 (gr_line (start 86.36 73.66) (end 86.36 154.94) (layer "Edge.Cuts") (width 0.1))
 (gr_line (start 154.94 154.94) (end 86.36 154.94) (layer "Edge.Cuts") (width 0.1))
 (gr_line (start 154.94 73.66) (end 154.94 154.94) (layer "Edge.Cuts") (width 0.1))
 (segment (start 91.44 122.595) (end 91.44 101.6) (width 0.25) (layer "F.Cu") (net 4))
 (segment (start 100.925 132.08) (end 91.44 122.595) (width 0.25) (layer "F.Cu") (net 4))
 (segment (start 147.74 94.4) (end 147.32 93.98) (width 0.25) (layer "F.Cu") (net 4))
 (segment (start 93.98 104.14) (end 96.52 104.14) (width 0.25) (layer "F.Cu") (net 4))
 (segment (start 96.52 91.44) (end 91.44 96.52) (width 0.25) (layer "F.Cu") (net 4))
 (segment (start 101.6 132.08) (end 100.925 132.08) (width 0.25) (layer "F.Cu") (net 4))
 (segment (start 91.44 96.52) (end 91.44 101.6) (width 0.25) (layer "F.Cu") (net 4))
 (segment (start 147.32 93.98) (end 144.78 91.44) (width 0.25) (layer "F.Cu") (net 4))
 (segment (start 144.78 91.44) (end 134.62 91.44) (width 0.25) (layer "F.Cu") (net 4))
 (segment (start 134.62 91.44) (end 135.295 91.44) (width 0.25) (layer "F.Cu") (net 4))
 (segment (start 147.74 111.3) (end 147.74 94.4) (width 0.25) (layer "F.Cu") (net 4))
 (segment (start 91.44 101.6) (end 93.98 104.14) (width 0.25) (layer "F.Cu") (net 4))
 (segment (start 123.2 135.905) (end 115.58 135.905) (width 0.25) (layer "B.Cu") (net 4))
 (segment (start 115.58 102.88) (end 97.78 102.88) (width 0.25) (layer "B.Cu") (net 4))
 (segment (start 115.58 138.445) (end 107.965 138.445) (width 0.25) (layer "B.Cu") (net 4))
 (segment (start 97.78 102.88) (end 96.52 104.14) (width 0.25) (layer "B.Cu") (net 4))
 (segment (start 132.08 91.44) (end 134.62 91.44) (width 0.25) (layer "B.Cu") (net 4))
 (segment (start 105.425 135.905) (end 101.6 132.08) (width 0.25) (layer "B.Cu") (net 4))
 (segment (start 115.58 135.905) (end 105.425 135.905) (width 0.25) (layer "B.Cu") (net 4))
 (segment (start 107.965 138.445) (end 104.14 134.62) (width 0.25) (layer "B.Cu") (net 4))
 (segment (start 122.075489 96.384511) (end 127.135489 96.384511) (width 0.25) (layer "B.Cu") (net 4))
 (segment (start 115.58 102.88) (end 122.075489 96.384511) (width 0.25) (layer "B.Cu") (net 4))
 (segment (start 123.2 138.445) (end 115.58 138.445) (width 0.25) (layer "B.Cu") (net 4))
 (segment (start 127.135489 96.384511) (end 132.08 91.44) (width 0.25) (layer "B.Cu") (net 4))
 (segment (start 97.79 92.71) (end 99.06 93.98) (width 0.25) (layer "F.Cu") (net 14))
 (segment (start 99.06 93.98) (end 101.6 93.98) (width 0.25) (layer "F.Cu") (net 14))
 (segment (start 101.6 93.98) (end 107.94 87.64) (width 0.25) (layer "F.Cu") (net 14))
 (segment (start 107.94 87.64) (end 115.58 87.64) (width 0.25) (layer "F.Cu") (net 14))
 (segment (start 134.62 92.44) (end 133.08 92.44) (width 0.25) (layer "F.Cu") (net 32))
 (segment (start 130.82 90.18) (end 123.2 90.18) (width 0.25) (layer "F.Cu") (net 32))
 (segment (start 133.08 92.44) (end 130.82 90.18) (width 0.25) (layer "F.Cu") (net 32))
 (segment (start 97.79 100.33) (end 107.94 90.18) (width 0.25) (layer "F.Cu") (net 11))
 (segment (start 107.94 90.18) (end 115.58 90.18) (width 0.25) (layer "F.Cu") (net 11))
 (segment (start 97.79 105.41) (end 97.79 100.33) (width 0.25) (layer "F.Cu") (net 11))
 (segment (start 123.92 93.44) (end 123.2 92.72) (width 0.25) (layer "F.Cu") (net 31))
 (segment (start 134.62 93.44) (end 123.92 93.44) (width 0.25) (layer "F.Cu") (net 31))
 (segment (start 97.195 78.74) (end 96.52 78.74) (width 0.25) (layer "F.Cu") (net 35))
 (segment (start 99.06 91.44) (end 99.06 80.605) (width 0.25) (layer "F.Cu") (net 35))
 (segment (start 99.06 80.605) (end 97.195 78.74) (width 0.25) (layer "F.Cu") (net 35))
 (segment (start 99.06 104.14) (end 99.06 111.76) (width 0.25) (layer "F.Cu") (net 12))
 (segment (start 99.06 111.76) (end 96.52 114.3) (width 0.25) (layer "F.Cu") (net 12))
 (segment (start 101.6 130.08) (end 112.295 130.08) (width 0.25) (layer "B.Cu") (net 3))
 (segment (start 112.295 130.08) (end 115.58 133.365) (width 0.25) (layer "B.Cu") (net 3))
 (segment (start 115.58 130.825) (end 111.76 127.005) (width 0.25) (layer "B.Cu") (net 2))
 (segment (start 113.02 118.12) (end 115.58 118.12) (width 0.25) (layer "B.Cu") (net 2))
 (segment (start 111.76 127.005) (end 111.76 119.38) (width 0.25) (layer "B.Cu") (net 2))
 (segment (start 111.76 119.38) (end 113.02 118.12) (width 0.25) (layer "B.Cu") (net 2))
 (segment (start 115.58 143.525) (end 116.865 142.24) (width 0.25) (layer "B.Cu") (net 6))
 (segment (start 116.865 142.24) (end 127 142.24) (width 0.25) (layer "B.Cu") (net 6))
 (segment (start 127 142.24) (end 132.08 137.16) (width 0.25) (layer "B.Cu") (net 6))
 (segment (start 132.08 127) (end 123.2 118.12) (width 0.25) (layer "B.Cu") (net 6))
 (segment (start 132.08 137.16) (end 132.08 127) (width 0.25) (layer "B.Cu") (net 6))
 (segment (start 125.74 115.58) (end 123.2 115.58) (width 0.25) (layer "F.Cu") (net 7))
 (segment (start 129.54 119.38) (end 125.74 115.58) (width 0.25) (layer "F.Cu") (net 7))
 (segment (start 123.2 143.525) (end 129.54 137.185) (width 0.25) (layer "F.Cu") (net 7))
 (segment (start 129.54 137.185) (end 129.54 119.38) (width 0.25) (layer "F.Cu") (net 7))
 (segment (start 123.2 130.825) (end 122.075489 129.700489) (width 0.25) (layer "F.Cu") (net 10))
 (segment (start 122.075489 129.695489) (end 119.38 127) (width 0.25) (layer "F.Cu") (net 10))
 (segment (start 119.38 116.86) (end 123.2 113.04) (width 0.25) (layer "F.Cu") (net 10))
 (segment (start 122.075489 129.700489) (end 122.075489 129.695489) (width 0.25) (layer "F.Cu") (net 10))
 (segment (start 119.38 127) (end 119.38 116.86) (width 0.25) (layer "F.Cu") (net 10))
 (segment (start 121.92 144.785) (end 123.2 146.065) (width 0.25) (layer "F.Cu") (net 1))
 (segment (start 122.734211 142.400489) (end 121.92 143.2147) (width 0.25) (layer "F.Cu") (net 1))
 (segment (start 102.595 115.3) (end 96.52 115.3) (width 0.25) (layer "F.Cu") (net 1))
 (segment (start 136.74 117.3) (end 136.74 135.04) (width 0.25) (layer "F.Cu") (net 1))
 (segment (start 125.715 146.065) (end 123.2 146.065) (width 0.25) (layer "F.Cu") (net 1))
 (segment (start 121.92 143.2147) (end 121.92 144.785) (width 0.25) (layer "F.Cu") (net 1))
 (segment (start 124.46 129.545) (end 124.46 141.629282) (width 0.25) (layer "F.Cu") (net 1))
 (segment (start 124.46 141.629282) (end 123.688793 142.400489) (width 0.25) (layer "F.Cu") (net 1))
 (segment (start 115.58 128.285) (end 102.595 115.3) (width 0.25) (layer "F.Cu") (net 1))
 (segment (start 136.74 135.04) (end 125.715 146.065) (width 0.25) (layer "F.Cu") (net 1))
 (segment (start 123.2 128.285) (end 124.46 129.545) (width 0.25) (layer "F.Cu") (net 1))
 (segment (start 123.688793 142.400489) (end 122.734211 142.400489) (width 0.25) (layer "F.Cu") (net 1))
 (segment (start 123.2 146.065) (end 115.58 146.065) (width 0.25) (layer "F.Cu") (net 1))
 (segment (start 88.9 98.027468) (end 88.9 86.36) (width 0.25) (layer "B.Cu") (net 1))
 (segment (start 97.12104 115.3) (end 97.269511 115.151529) (width 0.25) (layer "B.Cu") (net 1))
 (segment (start 97.269511 115.151529) (end 97.269511 106.396979) (width 0.25) (layer "B.Cu") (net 1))
 (segment (start 97.269511 106.396979) (end 88.9 98.027468) (width 0.25) (layer "B.Cu") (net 1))
 (segment (start 115.58 128.285) (end 123.2 128.285) (width 0.25) (layer "B.Cu") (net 1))
 (segment (start 95.52 79.74) (end 96.52 79.74) (width 0.25) (layer "B.Cu") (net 1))
 (segment (start 96.52 115.3) (end 97.12104 115.3) (width 0.25) (layer "B.Cu") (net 1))
 (segment (start 88.9 86.36) (end 95.52 79.74) (width 0.25) (layer "B.Cu") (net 1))
 (segment (start 134.62 95.44) (end 125.56 95.44) (width 0.25) (layer "F.Cu") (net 29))
 (segment (start 125.56 95.44) (end 123.2 97.8) (width 0.25) (layer "F.Cu") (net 29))
 (segment (start 134.62 94.44) (end 124.02 94.44) (width 0.25) (layer "F.Cu") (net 30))
 (segment (start 124.02 94.44) (end 123.2 95.26) (width 0.25) (layer "F.Cu") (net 30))
 (segment (start 101.6 129.08) (end 109.413722 129.08) (width 0.25) (layer "F.Cu") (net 8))
 (segment (start 115.114211 134.780489) (end 116.995489 134.780489) (width 0.25) (layer "F.Cu") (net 8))
 (segment (start 109.413722 129.08) (end 115.114211 134.780489) (width 0.25) (layer "F.Cu") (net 8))
 (segment (start 116.995489 134.780489) (end 123.2 140.985) (width 0.25) (layer "F.Cu") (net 8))
 (segment (start 114.585978 129.54) (end 119.375 129.54) (width 0.25) (layer "F.Cu") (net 9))
 (segment (start 113.125978 128.08) (end 114.585978 129.54) (width 0.25) (layer "F.Cu") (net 9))
 (segment (start 101.6 128.08) (end 113.125978 128.08) (width 0.25) (layer "F.Cu") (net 9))
 (segment (start 119.375 129.54) (end 123.2 133.365) (width 0.25) (layer "F.Cu") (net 9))
 (segment (start 101.6 131.08) (end 105.675 131.08) (width 0.25) (layer "F.Cu") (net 5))
 (segment (start 105.675 131.08) (end 115.58 140.985) (width 0.25) (layer "F.Cu") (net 5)))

